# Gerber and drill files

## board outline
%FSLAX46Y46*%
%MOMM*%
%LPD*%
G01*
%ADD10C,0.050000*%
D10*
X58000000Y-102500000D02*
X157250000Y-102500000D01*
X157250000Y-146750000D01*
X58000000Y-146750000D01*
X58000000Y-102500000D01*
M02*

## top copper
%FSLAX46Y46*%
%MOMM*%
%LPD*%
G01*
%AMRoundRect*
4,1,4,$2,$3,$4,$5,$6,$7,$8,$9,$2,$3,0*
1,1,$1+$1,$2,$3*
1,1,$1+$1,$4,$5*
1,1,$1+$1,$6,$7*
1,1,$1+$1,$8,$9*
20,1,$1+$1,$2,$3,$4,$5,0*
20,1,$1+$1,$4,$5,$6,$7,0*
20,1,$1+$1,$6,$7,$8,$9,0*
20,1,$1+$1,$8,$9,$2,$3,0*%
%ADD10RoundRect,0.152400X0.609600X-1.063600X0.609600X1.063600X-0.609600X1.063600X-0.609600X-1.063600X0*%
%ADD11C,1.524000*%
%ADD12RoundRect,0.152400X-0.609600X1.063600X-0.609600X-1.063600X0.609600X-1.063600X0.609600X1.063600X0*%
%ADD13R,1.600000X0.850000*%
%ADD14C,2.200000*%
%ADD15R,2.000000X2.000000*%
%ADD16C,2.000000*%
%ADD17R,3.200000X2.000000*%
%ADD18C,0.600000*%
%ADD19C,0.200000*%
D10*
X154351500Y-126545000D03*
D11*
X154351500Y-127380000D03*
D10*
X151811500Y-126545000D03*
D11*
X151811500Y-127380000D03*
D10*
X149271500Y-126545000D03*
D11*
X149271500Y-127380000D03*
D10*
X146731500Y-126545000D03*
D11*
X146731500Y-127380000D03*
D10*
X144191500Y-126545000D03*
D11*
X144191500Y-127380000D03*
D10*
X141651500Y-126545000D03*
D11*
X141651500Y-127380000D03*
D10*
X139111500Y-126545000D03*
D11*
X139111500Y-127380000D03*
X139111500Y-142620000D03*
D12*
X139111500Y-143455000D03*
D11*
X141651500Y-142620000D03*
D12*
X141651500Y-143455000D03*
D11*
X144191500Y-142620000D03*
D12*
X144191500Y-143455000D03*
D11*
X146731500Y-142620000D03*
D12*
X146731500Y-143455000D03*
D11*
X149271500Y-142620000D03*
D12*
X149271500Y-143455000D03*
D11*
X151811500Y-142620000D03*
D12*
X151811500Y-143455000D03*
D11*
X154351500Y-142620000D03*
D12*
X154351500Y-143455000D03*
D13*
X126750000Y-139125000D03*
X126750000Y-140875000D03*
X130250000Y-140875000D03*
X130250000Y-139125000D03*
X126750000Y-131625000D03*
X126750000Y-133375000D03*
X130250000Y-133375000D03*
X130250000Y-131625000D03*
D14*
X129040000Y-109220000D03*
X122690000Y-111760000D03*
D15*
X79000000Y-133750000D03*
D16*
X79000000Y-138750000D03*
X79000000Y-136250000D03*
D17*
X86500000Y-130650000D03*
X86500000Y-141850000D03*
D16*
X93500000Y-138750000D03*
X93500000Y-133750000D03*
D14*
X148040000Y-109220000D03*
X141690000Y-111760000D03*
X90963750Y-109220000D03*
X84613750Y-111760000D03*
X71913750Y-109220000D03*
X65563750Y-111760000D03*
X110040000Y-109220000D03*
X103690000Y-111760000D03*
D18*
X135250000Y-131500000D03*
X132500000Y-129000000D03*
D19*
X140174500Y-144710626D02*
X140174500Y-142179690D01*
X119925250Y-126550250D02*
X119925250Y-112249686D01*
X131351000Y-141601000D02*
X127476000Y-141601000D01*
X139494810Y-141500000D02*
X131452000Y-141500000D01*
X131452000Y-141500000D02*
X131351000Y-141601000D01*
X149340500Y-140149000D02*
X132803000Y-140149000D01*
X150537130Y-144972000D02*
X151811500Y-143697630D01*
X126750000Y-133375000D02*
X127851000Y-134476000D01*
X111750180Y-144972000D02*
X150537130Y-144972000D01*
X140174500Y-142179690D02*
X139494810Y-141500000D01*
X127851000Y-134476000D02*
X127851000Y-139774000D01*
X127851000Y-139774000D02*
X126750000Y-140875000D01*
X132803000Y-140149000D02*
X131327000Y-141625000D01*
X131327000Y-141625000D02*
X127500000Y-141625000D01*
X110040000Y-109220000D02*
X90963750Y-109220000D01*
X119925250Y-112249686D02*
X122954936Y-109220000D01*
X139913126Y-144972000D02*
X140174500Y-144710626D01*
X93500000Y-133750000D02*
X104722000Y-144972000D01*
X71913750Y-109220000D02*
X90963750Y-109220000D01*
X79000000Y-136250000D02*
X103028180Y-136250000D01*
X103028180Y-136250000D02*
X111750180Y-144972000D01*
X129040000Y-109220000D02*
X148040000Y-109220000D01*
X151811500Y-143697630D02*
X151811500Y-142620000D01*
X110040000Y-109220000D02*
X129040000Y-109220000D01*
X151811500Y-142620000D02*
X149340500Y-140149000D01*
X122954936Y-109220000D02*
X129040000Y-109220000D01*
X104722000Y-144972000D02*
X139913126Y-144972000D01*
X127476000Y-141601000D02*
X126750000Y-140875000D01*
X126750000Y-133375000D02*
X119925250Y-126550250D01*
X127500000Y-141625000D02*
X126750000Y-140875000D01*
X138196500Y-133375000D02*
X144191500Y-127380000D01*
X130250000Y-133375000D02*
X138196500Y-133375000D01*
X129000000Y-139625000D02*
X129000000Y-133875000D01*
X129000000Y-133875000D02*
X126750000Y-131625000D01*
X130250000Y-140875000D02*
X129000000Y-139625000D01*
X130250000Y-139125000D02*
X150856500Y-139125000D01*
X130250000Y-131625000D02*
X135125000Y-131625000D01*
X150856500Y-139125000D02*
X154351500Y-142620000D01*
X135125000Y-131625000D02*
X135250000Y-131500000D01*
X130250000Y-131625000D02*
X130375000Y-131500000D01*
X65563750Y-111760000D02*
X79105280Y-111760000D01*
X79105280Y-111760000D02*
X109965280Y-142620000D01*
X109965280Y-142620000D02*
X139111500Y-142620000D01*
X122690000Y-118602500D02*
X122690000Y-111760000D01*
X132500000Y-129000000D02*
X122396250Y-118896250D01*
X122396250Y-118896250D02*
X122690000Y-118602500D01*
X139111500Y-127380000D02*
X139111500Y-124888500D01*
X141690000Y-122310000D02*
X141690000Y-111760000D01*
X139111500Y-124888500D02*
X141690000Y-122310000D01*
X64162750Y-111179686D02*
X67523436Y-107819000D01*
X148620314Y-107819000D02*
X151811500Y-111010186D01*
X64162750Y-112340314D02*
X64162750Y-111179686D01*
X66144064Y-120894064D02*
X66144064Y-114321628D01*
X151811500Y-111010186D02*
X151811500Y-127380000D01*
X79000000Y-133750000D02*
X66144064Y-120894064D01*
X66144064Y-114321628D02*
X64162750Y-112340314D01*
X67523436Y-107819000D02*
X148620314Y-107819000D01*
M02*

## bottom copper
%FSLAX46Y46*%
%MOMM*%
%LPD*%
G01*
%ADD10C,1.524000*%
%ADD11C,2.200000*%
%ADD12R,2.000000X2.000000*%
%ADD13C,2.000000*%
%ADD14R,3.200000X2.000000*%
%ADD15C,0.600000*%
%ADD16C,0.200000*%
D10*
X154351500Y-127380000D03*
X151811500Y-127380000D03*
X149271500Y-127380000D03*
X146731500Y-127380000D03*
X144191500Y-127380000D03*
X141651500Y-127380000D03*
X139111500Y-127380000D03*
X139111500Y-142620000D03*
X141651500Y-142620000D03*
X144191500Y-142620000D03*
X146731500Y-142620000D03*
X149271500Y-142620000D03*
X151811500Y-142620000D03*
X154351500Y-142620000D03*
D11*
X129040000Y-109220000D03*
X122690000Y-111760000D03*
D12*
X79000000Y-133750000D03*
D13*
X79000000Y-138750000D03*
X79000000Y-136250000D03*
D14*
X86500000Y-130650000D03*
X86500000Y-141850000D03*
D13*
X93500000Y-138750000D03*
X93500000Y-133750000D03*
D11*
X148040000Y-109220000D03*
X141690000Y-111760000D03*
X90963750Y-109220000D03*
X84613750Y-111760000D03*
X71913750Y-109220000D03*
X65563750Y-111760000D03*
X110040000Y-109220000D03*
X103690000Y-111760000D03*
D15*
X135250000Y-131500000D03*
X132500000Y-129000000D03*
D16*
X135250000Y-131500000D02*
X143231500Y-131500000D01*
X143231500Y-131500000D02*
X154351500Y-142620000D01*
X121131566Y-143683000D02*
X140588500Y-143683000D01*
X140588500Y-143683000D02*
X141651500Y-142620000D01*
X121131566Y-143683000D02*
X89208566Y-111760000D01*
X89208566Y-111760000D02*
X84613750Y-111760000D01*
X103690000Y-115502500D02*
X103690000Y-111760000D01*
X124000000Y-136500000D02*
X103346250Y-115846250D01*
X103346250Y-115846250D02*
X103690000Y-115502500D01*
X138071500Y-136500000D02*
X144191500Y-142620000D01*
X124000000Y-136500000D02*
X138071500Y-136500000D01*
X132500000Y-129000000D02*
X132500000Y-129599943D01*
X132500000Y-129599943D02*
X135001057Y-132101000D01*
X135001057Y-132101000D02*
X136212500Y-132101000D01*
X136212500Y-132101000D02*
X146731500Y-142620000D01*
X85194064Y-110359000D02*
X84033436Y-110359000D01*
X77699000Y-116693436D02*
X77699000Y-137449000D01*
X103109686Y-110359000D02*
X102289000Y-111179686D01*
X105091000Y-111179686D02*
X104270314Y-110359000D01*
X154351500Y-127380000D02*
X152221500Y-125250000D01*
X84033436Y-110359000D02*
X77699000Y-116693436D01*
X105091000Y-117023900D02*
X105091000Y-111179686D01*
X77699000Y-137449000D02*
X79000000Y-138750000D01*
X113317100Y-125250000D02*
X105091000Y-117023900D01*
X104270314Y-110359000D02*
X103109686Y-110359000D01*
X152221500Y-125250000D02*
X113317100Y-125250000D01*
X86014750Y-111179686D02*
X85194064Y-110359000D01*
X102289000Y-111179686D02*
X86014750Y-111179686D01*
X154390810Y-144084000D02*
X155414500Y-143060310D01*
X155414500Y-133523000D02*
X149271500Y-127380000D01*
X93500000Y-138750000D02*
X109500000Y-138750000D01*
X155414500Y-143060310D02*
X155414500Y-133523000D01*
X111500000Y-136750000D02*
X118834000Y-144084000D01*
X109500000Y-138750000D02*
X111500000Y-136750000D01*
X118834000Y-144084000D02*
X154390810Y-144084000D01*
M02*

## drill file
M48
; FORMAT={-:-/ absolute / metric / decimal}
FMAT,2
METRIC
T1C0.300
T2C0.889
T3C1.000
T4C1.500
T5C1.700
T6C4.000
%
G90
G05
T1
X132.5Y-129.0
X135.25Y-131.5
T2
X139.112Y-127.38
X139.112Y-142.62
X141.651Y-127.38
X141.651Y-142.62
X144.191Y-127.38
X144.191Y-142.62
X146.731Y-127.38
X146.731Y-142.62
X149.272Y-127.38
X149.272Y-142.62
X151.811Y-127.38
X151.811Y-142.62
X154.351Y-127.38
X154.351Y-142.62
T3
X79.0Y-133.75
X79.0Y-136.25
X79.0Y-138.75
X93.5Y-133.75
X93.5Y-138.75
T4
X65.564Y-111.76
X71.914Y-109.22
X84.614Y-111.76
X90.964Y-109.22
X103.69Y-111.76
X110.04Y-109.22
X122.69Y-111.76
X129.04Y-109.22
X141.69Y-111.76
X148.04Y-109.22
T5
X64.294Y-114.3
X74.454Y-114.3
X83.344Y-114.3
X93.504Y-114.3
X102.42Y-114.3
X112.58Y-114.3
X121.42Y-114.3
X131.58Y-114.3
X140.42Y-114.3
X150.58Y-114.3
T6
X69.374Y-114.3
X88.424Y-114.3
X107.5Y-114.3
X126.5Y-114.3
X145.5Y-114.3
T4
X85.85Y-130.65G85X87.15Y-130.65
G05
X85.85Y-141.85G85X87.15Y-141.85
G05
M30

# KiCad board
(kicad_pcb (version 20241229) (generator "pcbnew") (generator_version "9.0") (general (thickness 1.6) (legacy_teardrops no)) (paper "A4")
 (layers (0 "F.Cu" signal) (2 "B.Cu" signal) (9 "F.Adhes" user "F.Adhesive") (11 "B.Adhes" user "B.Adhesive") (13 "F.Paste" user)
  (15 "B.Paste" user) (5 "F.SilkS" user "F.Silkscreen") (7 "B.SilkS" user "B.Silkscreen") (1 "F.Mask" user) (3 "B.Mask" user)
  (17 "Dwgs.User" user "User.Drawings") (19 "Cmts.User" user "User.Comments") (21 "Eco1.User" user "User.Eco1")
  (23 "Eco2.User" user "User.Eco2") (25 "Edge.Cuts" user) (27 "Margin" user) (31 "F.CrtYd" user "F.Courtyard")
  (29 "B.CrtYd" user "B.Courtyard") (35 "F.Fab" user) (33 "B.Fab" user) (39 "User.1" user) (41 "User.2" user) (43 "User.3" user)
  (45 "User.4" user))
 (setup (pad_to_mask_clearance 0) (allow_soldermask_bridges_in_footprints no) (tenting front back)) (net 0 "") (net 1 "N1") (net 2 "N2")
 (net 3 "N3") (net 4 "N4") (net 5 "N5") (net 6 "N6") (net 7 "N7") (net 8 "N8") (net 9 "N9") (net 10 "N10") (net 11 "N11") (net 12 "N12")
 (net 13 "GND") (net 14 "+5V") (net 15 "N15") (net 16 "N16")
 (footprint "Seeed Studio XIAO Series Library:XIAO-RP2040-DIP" (layer "F.Cu") (at 146.7315 135 -90)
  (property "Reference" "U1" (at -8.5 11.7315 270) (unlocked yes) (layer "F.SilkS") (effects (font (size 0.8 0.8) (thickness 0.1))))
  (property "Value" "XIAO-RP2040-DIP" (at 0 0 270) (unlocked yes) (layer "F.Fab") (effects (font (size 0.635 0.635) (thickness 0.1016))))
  (pad "1" smd roundrect (at -8.455 -7.62 90) (size 2.432 1.524) (layers "F.Cu" "F.Mask") (roundrect_rratio 0.1) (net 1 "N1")
   (thermal_bridge_angle 45))
  (pad "1" thru_hole circle (at -7.62 -7.62 90) (size 1.524 1.524) (drill 0.889) (layers "*.Cu" "*.Mask") (remove_unused_layers no)
   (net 1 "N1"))
  (pad "2" smd roundrect (at -8.455 -5.08 90) (size 2.432 1.524) (layers "F.Cu" "F.Mask") (roundrect_rratio 0.1) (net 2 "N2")
   (thermal_bridge_angle 45))
  (pad "2" thru_hole circle (at -7.62 -5.08 90) (size 1.524 1.524) (drill 0.889) (layers "*.Cu" "*.Mask") (remove_unused_layers no)
   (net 2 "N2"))
  (pad "3" smd roundrect (at -8.455 -2.54 90) (size 2.432 1.524) (layers "F.Cu" "F.Mask") (roundrect_rratio 0.1) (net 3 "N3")
   (thermal_bridge_angle 45))
  (pad "3" thru_hole circle (at -7.62 -2.54 90) (size 1.524 1.524) (drill 0.889) (layers "*.Cu" "*.Mask") (remove_unused_layers no)
   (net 3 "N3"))
  (pad "4" smd roundrect (at -8.455 0 90) (size 2.432 1.524) (layers "F.Cu" "F.Mask") (roundrect_rratio 0.1) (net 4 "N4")
   (thermal_bridge_angle 45))
  (pad "4" thru_hole circle (at -7.62 0 90) (size 1.524 1.524) (drill 0.889) (layers "*.Cu" "*.Mask") (remove_unused_layers no) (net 4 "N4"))
  (pad "5" smd roundrect (at -8.455 2.54 90) (size 2.432 1.524) (layers "F.Cu" "F.Mask") (roundrect_rratio 0.1) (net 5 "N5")
   (thermal_bridge_angle 45))
  (pad "5" thru_hole circle (at -7.62 2.54 90) (size 1.524 1.524) (drill 0.889) (layers "*.Cu" "*.Mask") (remove_unused_layers no)
   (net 5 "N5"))
  (pad "6" smd roundrect (at -8.455 5.08 90) (size 2.432 1.524) (layers "F.Cu" "F.Mask") (roundrect_rratio 0.1) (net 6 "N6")
   (thermal_bridge_angle 45))
  (pad "6" thru_hole circle (at -7.62 5.08 90) (size 1.524 1.524) (drill 0.889) (layers "*.Cu" "*.Mask") (remove_unused_layers no)
   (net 6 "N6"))
  (pad "7" smd roundrect (at -8.455 7.62 90) (size 2.432 1.524) (layers "F.Cu" "F.Mask") (roundrect_rratio 0.1) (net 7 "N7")
   (thermal_bridge_angle 45))
  (pad "7" thru_hole circle (at -7.62 7.62 90) (size 1.524 1.524) (drill 0.889) (layers "*.Cu" "*.Mask") (remove_unused_layers no)
   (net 7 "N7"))
  (pad "8" thru_hole circle (at 7.62 7.62 270) (size 1.524 1.524) (drill 0.889) (layers "*.Cu" "*.Mask") (remove_unused_layers no)
   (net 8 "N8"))
  (pad "8" smd roundrect (at 8.455 7.62 270) (size 2.432 1.524) (layers "F.Cu" "F.Mask") (roundrect_rratio 0.1) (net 8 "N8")
   (thermal_bridge_angle 45))
  (pad "9" thru_hole circle (at 7.62 5.08 270) (size 1.524 1.524) (drill 0.889) (layers "*.Cu" "*.Mask") (remove_unused_layers no)
   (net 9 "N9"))
  (pad "9" smd roundrect (at 8.455 5.08 270) (size 2.432 1.524) (layers "F.Cu" "F.Mask") (roundrect_rratio 0.1) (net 9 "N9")
   (thermal_bridge_angle 45))
  (pad "10" thru_hole circle (at 7.62 2.54 270) (size 1.524 1.524) (drill 0.889) (layers "*.Cu" "*.Mask") (remove_unused_layers no)
   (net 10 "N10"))
  (pad "10" smd roundrect (at 8.455 2.54 270) (size 2.432 1.524) (layers "F.Cu" "F.Mask") (roundrect_rratio 0.1) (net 10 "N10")
   (thermal_bridge_angle 45))
  (pad "11" thru_hole circle (at 7.62 0 270) (size 1.524 1.524) (drill 0.889) (layers "*.Cu" "*.Mask") (remove_unused_layers no)
   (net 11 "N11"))
  (pad "11" smd roundrect (at 8.455 0 270) (size 2.432 1.524) (layers "F.Cu" "F.Mask") (roundrect_rratio 0.1) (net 11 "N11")
   (thermal_bridge_angle 45))
  (pad "12" thru_hole circle (at 7.62 -2.54 270) (size 1.524 1.524) (drill 0.889) (layers "*.Cu" "*.Mask") (remove_unused_layers no)
   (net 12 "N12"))
  (pad "12" smd roundrect (at 8.455 -2.54 270) (size 2.432 1.524) (layers "F.Cu" "F.Mask") (roundrect_rratio 0.1) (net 12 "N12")
   (thermal_bridge_angle 45))
  (pad "13" thru_hole circle (at 7.62 -5.08 270) (size 1.524 1.524) (drill 0.889) (layers "*.Cu" "*.Mask") (remove_unused_layers no)
   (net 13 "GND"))
  (pad "13" smd roundrect (at 8.455 -5.08 270) (size 2.432 1.524) (layers "F.Cu" "F.Mask") (roundrect_rratio 0.1) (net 13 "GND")
   (thermal_bridge_angle 45))
  (pad "14" thru_hole circle (at 7.62 -7.62 270) (size 1.524 1.524) (drill 0.889) (layers "*.Cu" "*.Mask") (remove_unused_layers no)
   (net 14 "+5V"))
  (pad "14" smd roundrect (at 8.455 -7.62 270) (size 2.432 1.524) (layers "F.Cu" "F.Mask") (roundrect_rratio 0.1) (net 14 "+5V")
   (thermal_bridge_angle 45)))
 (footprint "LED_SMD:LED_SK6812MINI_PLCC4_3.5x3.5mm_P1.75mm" (layer "F.Cu") (at 128.5 140)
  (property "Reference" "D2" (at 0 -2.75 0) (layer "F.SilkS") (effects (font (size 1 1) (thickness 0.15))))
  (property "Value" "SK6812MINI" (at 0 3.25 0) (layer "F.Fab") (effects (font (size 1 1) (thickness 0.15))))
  (pad "1" smd rect (at -1.75 -0.875) (size 1.6 0.85) (layers "F.Cu" "F.Mask" "F.Paste") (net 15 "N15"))
  (pad "2" smd rect (at -1.75 0.875) (size 1.6 0.85) (layers "F.Cu" "F.Mask" "F.Paste") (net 13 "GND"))
  (pad "3" smd rect (at 1.75 0.875) (size 1.6 0.85) (layers "F.Cu" "F.Mask" "F.Paste") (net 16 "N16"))
  (pad "4" smd rect (at 1.75 -0.875) (size 1.6 0.85) (layers "F.Cu" "F.Mask" "F.Paste") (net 14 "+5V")))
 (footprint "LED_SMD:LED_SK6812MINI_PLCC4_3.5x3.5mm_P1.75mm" (layer "F.Cu") (at 128.5 132.5)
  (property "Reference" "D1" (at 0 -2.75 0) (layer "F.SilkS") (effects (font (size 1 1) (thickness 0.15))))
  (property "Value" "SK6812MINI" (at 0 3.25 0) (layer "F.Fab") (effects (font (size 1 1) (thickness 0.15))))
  (pad "1" smd rect (at -1.75 -0.875) (size 1.6 0.85) (layers "F.Cu" "F.Mask" "F.Paste") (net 16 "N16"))
  (pad "2" smd rect (at -1.75 0.875) (size 1.6 0.85) (layers "F.Cu" "F.Mask" "F.Paste") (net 13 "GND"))
  (pad "3" smd rect (at 1.75 0.875) (size 1.6 0.85) (layers "F.Cu" "F.Mask" "F.Paste") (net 5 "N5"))
  (pad "4" smd rect (at 1.75 -0.875) (size 1.6 0.85) (layers "F.Cu" "F.Mask" "F.Paste") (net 14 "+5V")))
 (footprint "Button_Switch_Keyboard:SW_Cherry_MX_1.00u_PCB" (layer "F.Cu") (at 129.04 109.22)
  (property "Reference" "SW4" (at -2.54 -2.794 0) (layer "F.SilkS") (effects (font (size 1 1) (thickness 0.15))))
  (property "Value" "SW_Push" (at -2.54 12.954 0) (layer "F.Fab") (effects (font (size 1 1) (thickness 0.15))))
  (pad "" np_thru_hole circle (at -7.62 5.08) (size 1.7 1.7) (drill 1.7) (layers "*.Cu" "*.Mask"))
  (pad "" np_thru_hole circle (at -2.54 5.08) (size 4 4) (drill 4) (layers "*.Cu" "*.Mask"))
  (pad "" np_thru_hole circle (at 2.54 5.08) (size 1.7 1.7) (drill 1.7) (layers "*.Cu" "*.Mask"))
  (pad "1" thru_hole circle (at 0 0) (size 2.2 2.2) (drill 1.5) (layers "*.Cu" "*.Mask") (remove_unused_layers no) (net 13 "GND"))
  (pad "2" thru_hole circle (at -6.35 2.54) (size 2.2 2.2) (drill 1.5) (layers "*.Cu" "*.Mask") (remove_unused_layers no) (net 11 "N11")))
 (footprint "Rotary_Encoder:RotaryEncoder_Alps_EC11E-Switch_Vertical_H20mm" (layer "F.Cu") (at 79 133.75)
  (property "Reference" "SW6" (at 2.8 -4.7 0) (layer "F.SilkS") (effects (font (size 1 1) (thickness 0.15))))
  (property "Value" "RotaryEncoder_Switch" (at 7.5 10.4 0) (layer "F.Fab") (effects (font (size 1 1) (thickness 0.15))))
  (pad "A" thru_hole rect (at 0 0) (size 2 2) (drill 1) (layers "*.Cu" "*.Mask") (remove_unused_layers no) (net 2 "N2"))
  (pad "B" thru_hole circle (at 0 5) (size 2 2) (drill 1) (layers "*.Cu" "*.Mask") (remove_unused_layers no) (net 1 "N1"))
  (pad "C" thru_hole circle (at 0 2.5) (size 2 2) (drill 1) (layers "*.Cu" "*.Mask") (remove_unused_layers no) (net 13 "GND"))
  (pad "MP" thru_hole rect (at 7.5 -3.1) (size 3.2 2) (drill oval 2.8 1.5) (layers "*.Cu" "*.Mask") (remove_unused_layers no))
  (pad "MP" thru_hole rect (at 7.5 8.1) (size 3.2 2) (drill oval 2.8 1.5) (layers "*.Cu" "*.Mask") (remove_unused_layers no))
  (pad "S1" thru_hole circle (at 14.5 5) (size 2 2) (drill 1) (layers "*.Cu" "*.Mask") (remove_unused_layers no) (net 3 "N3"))
  (pad "S2" thru_hole circle (at 14.5 0) (size 2 2) (drill 1) (layers "*.Cu" "*.Mask") (remove_unused_layers no) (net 13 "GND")))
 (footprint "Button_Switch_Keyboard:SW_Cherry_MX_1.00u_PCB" (layer "F.Cu") (at 148.04 109.22)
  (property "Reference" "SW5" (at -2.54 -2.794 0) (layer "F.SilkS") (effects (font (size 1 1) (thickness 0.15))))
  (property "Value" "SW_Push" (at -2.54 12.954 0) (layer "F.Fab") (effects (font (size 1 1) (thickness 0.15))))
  (pad "" np_thru_hole circle (at -7.62 5.08) (size 1.7 1.7) (drill 1.7) (layers "*.Cu" "*.Mask"))
  (pad "" np_thru_hole circle (at -2.54 5.08) (size 4 4) (drill 4) (layers "*.Cu" "*.Mask"))
  (pad "" np_thru_hole circle (at 2.54 5.08) (size 1.7 1.7) (drill 1.7) (layers "*.Cu" "*.Mask"))
  (pad "1" thru_hole circle (at 0 0) (size 2.2 2.2) (drill 1.5) (layers "*.Cu" "*.Mask") (remove_unused_layers no) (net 13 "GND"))
  (pad "2" thru_hole circle (at -6.35 2.54) (size 2.2 2.2) (drill 1.5) (layers "*.Cu" "*.Mask") (remove_unused_layers no) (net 7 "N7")))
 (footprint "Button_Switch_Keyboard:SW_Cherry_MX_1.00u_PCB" (layer "F.Cu") (at 90.96375 109.22)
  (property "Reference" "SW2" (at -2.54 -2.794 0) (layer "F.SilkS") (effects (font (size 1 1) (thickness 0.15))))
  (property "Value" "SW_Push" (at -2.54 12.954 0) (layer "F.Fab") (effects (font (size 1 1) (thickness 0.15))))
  (pad "" np_thru_hole circle (at -7.62 5.08) (size 1.7 1.7) (drill 1.7) (layers "*.Cu" "*.Mask"))
  (pad "" np_thru_hole circle (at -2.54 5.08) (size 4 4) (drill 4) (layers "*.Cu" "*.Mask"))
  (pad "" np_thru_hole circle (at 2.54 5.08) (size 1.7 1.7) (drill 1.7) (layers "*.Cu" "*.Mask"))
  (pad "1" thru_hole circle (at 0 0) (size 2.2 2.2) (drill 1.5) (layers "*.Cu" "*.Mask") (remove_unused_layers no) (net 13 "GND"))
  (pad "2" thru_hole circle (at -6.35 2.54) (size 2.2 2.2) (drill 1.5) (layers "*.Cu" "*.Mask") (remove_unused_layers no) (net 9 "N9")))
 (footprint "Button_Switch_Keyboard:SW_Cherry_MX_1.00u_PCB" (layer "F.Cu") (at 71.91375 109.22)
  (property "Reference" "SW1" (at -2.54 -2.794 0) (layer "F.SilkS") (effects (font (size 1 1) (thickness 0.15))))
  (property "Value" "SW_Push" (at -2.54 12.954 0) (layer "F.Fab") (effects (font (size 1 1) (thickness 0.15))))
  (pad "" np_thru_hole circle (at -7.62 5.08) (size 1.7 1.7) (drill 1.7) (layers "*.Cu" "*.Mask"))
  (pad "" np_thru_hole circle (at -2.54 5.08) (size 4 4) (drill 4) (layers "*.Cu" "*.Mask"))
  (pad "" np_thru_hole circle (at 2.54 5.08) (size 1.7 1.7) (drill 1.7) (layers "*.Cu" "*.Mask"))
  (pad "1" thru_hole circle (at 0 0) (size 2.2 2.2) (drill 1.5) (layers "*.Cu" "*.Mask") (remove_unused_layers no) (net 13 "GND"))
  (pad "2" thru_hole circle (at -6.35 2.54) (size 2.2 2.2) (drill 1.5) (layers "*.Cu" "*.Mask") (remove_unused_layers no) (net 8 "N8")))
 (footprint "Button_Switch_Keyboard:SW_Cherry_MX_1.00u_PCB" (layer "F.Cu") (at 110.04 109.22)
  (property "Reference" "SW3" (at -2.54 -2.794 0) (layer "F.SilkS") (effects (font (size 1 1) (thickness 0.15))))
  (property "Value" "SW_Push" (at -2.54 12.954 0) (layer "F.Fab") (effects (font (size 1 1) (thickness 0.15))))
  (pad "" np_thru_hole circle (at -7.62 5.08) (size 1.7 1.7) (drill 1.7) (layers "*.Cu" "*.Mask"))
  (pad "" np_thru_hole circle (at -2.54 5.08) (size 4 4) (drill 4) (layers "*.Cu" "*.Mask"))
  (pad "" np_thru_hole circle (at 2.54 5.08) (size 1.7 1.7) (drill 1.7) (layers "*.Cu" "*.Mask"))
  (pad "1" thru_hole circle (at 0 0) (size 2.2 2.2) (drill 1.5) (layers "*.Cu" "*.Mask") (remove_unused_layers no) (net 13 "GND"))
  (pad "2" thru_hole circle (at -6.35 2.54) (size 2.2 2.2) (drill 1.5) (layers "*.Cu" "*.Mask") (remove_unused_layers no) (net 10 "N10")))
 (gr_rect (start 58 102.5) (end 157.25 146.75) (stroke (width 0.05) (type default)) (fill no) (layer "Edge.Cuts"))
 (segment (start 140.1745 144.710626) (end 140.1745 142.17969) (width 0.2) (layer "F.Cu") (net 13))
 (segment (start 119.92525 126.55025) (end 119.92525 112.249686) (width 0.2) (layer "F.Cu") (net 13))
 (segment (start 131.351 141.601) (end 127.476 141.601) (width 0.2) (layer "F.Cu") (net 13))
 (segment (start 139.49481 141.5) (end 131.452 141.5) (width 0.2) (layer "F.Cu") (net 13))
 (segment (start 131.452 141.5) (end 131.351 141.601) (width 0.2) (layer "F.Cu") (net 13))
 (segment (start 149.3405 140.149) (end 132.803 140.149) (width 0.2) (layer "F.Cu") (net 13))
 (segment (start 150.53713 144.972) (end 151.8115 143.69763) (width 0.2) (layer "F.Cu") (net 13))
 (segment (start 126.75 133.375) (end 127.851 134.476) (width 0.2) (layer "F.Cu") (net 13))
 (segment (start 111.75018 144.972) (end 150.53713 144.972) (width 0.2) (layer "F.Cu") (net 13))
 (segment (start 140.1745 142.17969) (end 139.49481 141.5) (width 0.2) (layer "F.Cu") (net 13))
 (segment (start 127.851 134.476) (end 127.851 139.774) (width 0.2) (layer "F.Cu") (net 13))
 (segment (start 127.851 139.774) (end 126.75 140.875) (width 0.2) (layer "F.Cu") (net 13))
 (segment (start 132.803 140.149) (end 131.327 141.625) (width 0.2) (layer "F.Cu") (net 13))
 (segment (start 131.327 141.625) (end 127.5 141.625) (width 0.2) (layer "F.Cu") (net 13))
 (segment (start 110.04 109.22) (end 90.96375 109.22) (width 0.2) (layer "F.Cu") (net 13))
 (segment (start 119.92525 112.249686) (end 122.954936 109.22) (width 0.2) (layer "F.Cu") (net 13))
 (segment (start 139.913126 144.972) (end 140.1745 144.710626) (width 0.2) (layer "F.Cu") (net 13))
 (segment (start 93.5 133.75) (end 104.722 144.972) (width 0.2) (layer "F.Cu") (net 13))
 (segment (start 71.91375 109.22) (end 90.96375 109.22) (width 0.2) (layer "F.Cu") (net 13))
 (segment (start 79 136.25) (end 103.02818 136.25) (width 0.2) (layer "F.Cu") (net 13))
 (segment (start 103.02818 136.25) (end 111.75018 144.972) (width 0.2) (layer "F.Cu") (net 13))
 (segment (start 129.04 109.22) (end 148.04 109.22) (width 0.2) (layer "F.Cu") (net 13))
 (segment (start 151.8115 143.69763) (end 151.8115 142.62) (width 0.2) (layer "F.Cu") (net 13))
 (segment (start 110.04 109.22) (end 129.04 109.22) (width 0.2) (layer "F.Cu") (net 13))
 (segment (start 151.8115 142.62) (end 149.3405 140.149) (width 0.2) (layer "F.Cu") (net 13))
 (segment (start 122.954936 109.22) (end 129.04 109.22) (width 0.2) (layer "F.Cu") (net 13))
 (segment (start 104.722 144.972) (end 139.913126 144.972) (width 0.2) (layer "F.Cu") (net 13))
 (segment (start 127.476 141.601) (end 126.75 140.875) (width 0.2) (layer "F.Cu") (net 13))
 (segment (start 126.75 133.375) (end 119.92525 126.55025) (width 0.2) (layer "F.Cu") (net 13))
 (segment (start 127.5 141.625) (end 126.75 140.875) (width 0.2) (layer "F.Cu") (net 13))
 (segment (start 138.1965 133.375) (end 144.1915 127.38) (width 0.2) (layer "F.Cu") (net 5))
 (segment (start 130.25 133.375) (end 138.1965 133.375) (width 0.2) (layer "F.Cu") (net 5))
 (segment (start 129 139.625) (end 129 133.875) (width 0.2) (layer "F.Cu") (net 16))
 (segment (start 129 133.875) (end 126.75 131.625) (width 0.2) (layer "F.Cu") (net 16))
 (segment (start 130.25 140.875) (end 129 139.625) (width 0.2) (layer "F.Cu") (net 16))
 (segment (start 130.25 139.125) (end 150.8565 139.125) (width 0.2) (layer "F.Cu") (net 14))
 (segment (start 130.25 131.625) (end 135.125 131.625) (width 0.2) (layer "F.Cu") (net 14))
 (segment (start 150.8565 139.125) (end 154.3515 142.62) (width 0.2) (layer "F.Cu") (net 14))
 (segment (start 135.125 131.625) (end 135.25 131.5) (width 0.2) (layer "F.Cu") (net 14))
 (segment (start 130.25 131.625) (end 130.375 131.5) (width 0.2) (layer "F.Cu") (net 14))
 (via (at 135.25 131.5) (size 0.6) (drill 0.3) (layers "F.Cu" "B.Cu") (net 14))
 (segment (start 135.25 131.5) (end 143.2315 131.5) (width 0.2) (layer "B.Cu") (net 14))
 (segment (start 143.2315 131.5) (end 154.3515 142.62) (width 0.2) (layer "B.Cu") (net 14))
 (segment (start 65.56375 111.76) (end 79.10528 111.76) (width 0.2) (layer "F.Cu") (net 8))
 (segment (start 79.10528 111.76) (end 109.96528 142.62) (width 0.2) (layer "F.Cu") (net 8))
 (segment (start 109.96528 142.62) (end 139.1115 142.62) (width 0.2) (layer "F.Cu") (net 8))
 (segment (start 121.131566 143.683) (end 140.5885 143.683) (width 0.2) (layer "B.Cu") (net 9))
 (segment (start 140.5885 143.683) (end 141.6515 142.62) (width 0.2) (layer "B.Cu") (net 9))
 (segment (start 121.131566 143.683) (end 89.208566 111.76) (width 0.2) (layer "B.Cu") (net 9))
 (segment (start 89.208566 111.76) (end 84.61375 111.76) (width 0.2) (layer "B.Cu") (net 9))
 (segment (start 103.69 115.5025) (end 103.69 111.76) (width 0.2) (layer "B.Cu") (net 10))
 (segment (start 124 136.5) (end 103.34625 115.84625) (width 0.2) (layer "B.Cu") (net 10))
 (segment (start 103.34625 115.84625) (end 103.69 115.5025) (width 0.2) (layer "B.Cu") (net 10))
 (segment (start 138.0715 136.5) (end 144.1915 142.62) (width 0.2) (layer "B.Cu") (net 10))
 (segment (start 124 136.5) (end 138.0715 136.5) (width 0.2) (layer "B.Cu") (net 10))
 (segment (start 122.69 118.6025) (end 122.69 111.76) (width 0.2) (layer "F.Cu") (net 11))
 (segment (start 132.5 129) (end 122.39625 118.89625) (width 0.2) (layer "F.Cu") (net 11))
 (segment (start 122.39625 118.89625) (end 122.69 118.6025) (width 0.2) (layer "F.Cu") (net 11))
 (via (at 132.5 129) (size 0.6) (drill 0.3) (layers "F.Cu" "B.Cu") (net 11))
 (segment (start 132.5 129) (end 132.5 129.599943) (width 0.2) (layer "B.Cu") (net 11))
 (segment (start 132.5 129.599943) (end 135.001057 132.101) (width 0.2) (layer "B.Cu") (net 11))
 (segment (start 135.001057 132.101) (end 136.2125 132.101) (width 0.2) (layer "B.Cu") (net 11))
 (segment (start 136.2125 132.101) (end 146.7315 142.62) (width 0.2) (layer "B.Cu") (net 11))
 (segment (start 85.194064 110.359) (end 84.033436 110.359) (width 0.2) (layer "B.Cu") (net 1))
 (segment (start 77.699 116.693436) (end 77.699 137.449) (width 0.2) (layer "B.Cu") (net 1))
 (segment (start 103.109686 110.359) (end 102.289 111.179686) (width 0.2) (layer "B.Cu") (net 1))
 (segment (start 105.091 111.179686) (end 104.270314 110.359) (width 0.2) (layer "B.Cu") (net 1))
 (segment (start 154.3515 127.38) (end 152.2215 125.25) (width 0.2) (layer "B.Cu") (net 1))
 (segment (start 84.033436 110.359) (end 77.699 116.693436) (width 0.2) (layer "B.Cu") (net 1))
 (segment (start 105.091 117.0239) (end 105.091 111.179686) (width 0.2) (layer "B.Cu") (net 1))
 (segment (start 77.699 137.449) (end 79 138.75) (width 0.2) (layer "B.Cu") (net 1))
 (segment (start 113.3171 125.25) (end 105.091 117.0239) (width 0.2) (layer "B.Cu") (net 1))
 (segment (start 104.270314 110.359) (end 103.109686 110.359) (width 0.2) (layer "B.Cu") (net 1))
 (segment (start 152.2215 125.25) (end 113.3171 125.25) (width 0.2) (layer "B.Cu") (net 1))
 (segment (start 86.01475 111.179686) (end 85.194064 110.359) (width 0.2) (layer "B.Cu") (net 1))
 (segment (start 102.289 111.179686) (end 86.01475 111.179686) (width 0.2) (layer "B.Cu") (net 1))
 (segment (start 154.39081 144.084) (end 155.4145 143.06031) (width 0.2) (layer "B.Cu") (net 3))
 (segment (start 155.4145 133.523) (end 149.2715 127.38) (width 0.2) (layer "B.Cu") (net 3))
 (segment (start 93.5 138.75) (end 109.5 138.75) (width 0.2) (layer "B.Cu") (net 3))
 (segment (start 155.4145 143.06031) (end 155.4145 133.523) (width 0.2) (layer "B.Cu") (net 3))
 (segment (start 111.5 136.75) (end 118.834 144.084) (width 0.2) (layer "B.Cu") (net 3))
 (segment (start 109.5 138.75) (end 111.5 136.75) (width 0.2) (layer "B.Cu") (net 3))
 (segment (start 118.834 144.084) (end 154.39081 144.084) (width 0.2) (layer "B.Cu") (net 3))
 (segment (start 139.1115 127.38) (end 139.1115 124.8885) (width 0.2) (layer "F.Cu") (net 7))
 (segment (start 141.69 122.31) (end 141.69 111.76) (width 0.2) (layer "F.Cu") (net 7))
 (segment (start 139.1115 124.8885) (end 141.69 122.31) (width 0.2) (layer "F.Cu") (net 7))
 (segment (start 64.16275 111.179686) (end 67.523436 107.819) (width 0.2) (layer "F.Cu") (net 2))
 (segment (start 148.620314 107.819) (end 151.8115 111.010186) (width 0.2) (layer "F.Cu") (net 2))
 (segment (start 64.16275 112.340314) (end 64.16275 111.179686) (width 0.2) (layer "F.Cu") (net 2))
 (segment (start 66.144064 120.894064) (end 66.144064 114.321628) (width 0.2) (layer "F.Cu") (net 2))
 (segment (start 151.8115 111.010186) (end 151.8115 127.38) (width 0.2) (layer "F.Cu") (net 2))
 (segment (start 79 133.75) (end 66.144064 120.894064) (width 0.2) (layer "F.Cu") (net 2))
 (segment (start 66.144064 114.321628) (end 64.16275 112.340314) (width 0.2) (layer "F.Cu") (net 2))
 (segment (start 67.523436 107.819) (end 148.620314 107.819) (width 0.2) (layer "F.Cu") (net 2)))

